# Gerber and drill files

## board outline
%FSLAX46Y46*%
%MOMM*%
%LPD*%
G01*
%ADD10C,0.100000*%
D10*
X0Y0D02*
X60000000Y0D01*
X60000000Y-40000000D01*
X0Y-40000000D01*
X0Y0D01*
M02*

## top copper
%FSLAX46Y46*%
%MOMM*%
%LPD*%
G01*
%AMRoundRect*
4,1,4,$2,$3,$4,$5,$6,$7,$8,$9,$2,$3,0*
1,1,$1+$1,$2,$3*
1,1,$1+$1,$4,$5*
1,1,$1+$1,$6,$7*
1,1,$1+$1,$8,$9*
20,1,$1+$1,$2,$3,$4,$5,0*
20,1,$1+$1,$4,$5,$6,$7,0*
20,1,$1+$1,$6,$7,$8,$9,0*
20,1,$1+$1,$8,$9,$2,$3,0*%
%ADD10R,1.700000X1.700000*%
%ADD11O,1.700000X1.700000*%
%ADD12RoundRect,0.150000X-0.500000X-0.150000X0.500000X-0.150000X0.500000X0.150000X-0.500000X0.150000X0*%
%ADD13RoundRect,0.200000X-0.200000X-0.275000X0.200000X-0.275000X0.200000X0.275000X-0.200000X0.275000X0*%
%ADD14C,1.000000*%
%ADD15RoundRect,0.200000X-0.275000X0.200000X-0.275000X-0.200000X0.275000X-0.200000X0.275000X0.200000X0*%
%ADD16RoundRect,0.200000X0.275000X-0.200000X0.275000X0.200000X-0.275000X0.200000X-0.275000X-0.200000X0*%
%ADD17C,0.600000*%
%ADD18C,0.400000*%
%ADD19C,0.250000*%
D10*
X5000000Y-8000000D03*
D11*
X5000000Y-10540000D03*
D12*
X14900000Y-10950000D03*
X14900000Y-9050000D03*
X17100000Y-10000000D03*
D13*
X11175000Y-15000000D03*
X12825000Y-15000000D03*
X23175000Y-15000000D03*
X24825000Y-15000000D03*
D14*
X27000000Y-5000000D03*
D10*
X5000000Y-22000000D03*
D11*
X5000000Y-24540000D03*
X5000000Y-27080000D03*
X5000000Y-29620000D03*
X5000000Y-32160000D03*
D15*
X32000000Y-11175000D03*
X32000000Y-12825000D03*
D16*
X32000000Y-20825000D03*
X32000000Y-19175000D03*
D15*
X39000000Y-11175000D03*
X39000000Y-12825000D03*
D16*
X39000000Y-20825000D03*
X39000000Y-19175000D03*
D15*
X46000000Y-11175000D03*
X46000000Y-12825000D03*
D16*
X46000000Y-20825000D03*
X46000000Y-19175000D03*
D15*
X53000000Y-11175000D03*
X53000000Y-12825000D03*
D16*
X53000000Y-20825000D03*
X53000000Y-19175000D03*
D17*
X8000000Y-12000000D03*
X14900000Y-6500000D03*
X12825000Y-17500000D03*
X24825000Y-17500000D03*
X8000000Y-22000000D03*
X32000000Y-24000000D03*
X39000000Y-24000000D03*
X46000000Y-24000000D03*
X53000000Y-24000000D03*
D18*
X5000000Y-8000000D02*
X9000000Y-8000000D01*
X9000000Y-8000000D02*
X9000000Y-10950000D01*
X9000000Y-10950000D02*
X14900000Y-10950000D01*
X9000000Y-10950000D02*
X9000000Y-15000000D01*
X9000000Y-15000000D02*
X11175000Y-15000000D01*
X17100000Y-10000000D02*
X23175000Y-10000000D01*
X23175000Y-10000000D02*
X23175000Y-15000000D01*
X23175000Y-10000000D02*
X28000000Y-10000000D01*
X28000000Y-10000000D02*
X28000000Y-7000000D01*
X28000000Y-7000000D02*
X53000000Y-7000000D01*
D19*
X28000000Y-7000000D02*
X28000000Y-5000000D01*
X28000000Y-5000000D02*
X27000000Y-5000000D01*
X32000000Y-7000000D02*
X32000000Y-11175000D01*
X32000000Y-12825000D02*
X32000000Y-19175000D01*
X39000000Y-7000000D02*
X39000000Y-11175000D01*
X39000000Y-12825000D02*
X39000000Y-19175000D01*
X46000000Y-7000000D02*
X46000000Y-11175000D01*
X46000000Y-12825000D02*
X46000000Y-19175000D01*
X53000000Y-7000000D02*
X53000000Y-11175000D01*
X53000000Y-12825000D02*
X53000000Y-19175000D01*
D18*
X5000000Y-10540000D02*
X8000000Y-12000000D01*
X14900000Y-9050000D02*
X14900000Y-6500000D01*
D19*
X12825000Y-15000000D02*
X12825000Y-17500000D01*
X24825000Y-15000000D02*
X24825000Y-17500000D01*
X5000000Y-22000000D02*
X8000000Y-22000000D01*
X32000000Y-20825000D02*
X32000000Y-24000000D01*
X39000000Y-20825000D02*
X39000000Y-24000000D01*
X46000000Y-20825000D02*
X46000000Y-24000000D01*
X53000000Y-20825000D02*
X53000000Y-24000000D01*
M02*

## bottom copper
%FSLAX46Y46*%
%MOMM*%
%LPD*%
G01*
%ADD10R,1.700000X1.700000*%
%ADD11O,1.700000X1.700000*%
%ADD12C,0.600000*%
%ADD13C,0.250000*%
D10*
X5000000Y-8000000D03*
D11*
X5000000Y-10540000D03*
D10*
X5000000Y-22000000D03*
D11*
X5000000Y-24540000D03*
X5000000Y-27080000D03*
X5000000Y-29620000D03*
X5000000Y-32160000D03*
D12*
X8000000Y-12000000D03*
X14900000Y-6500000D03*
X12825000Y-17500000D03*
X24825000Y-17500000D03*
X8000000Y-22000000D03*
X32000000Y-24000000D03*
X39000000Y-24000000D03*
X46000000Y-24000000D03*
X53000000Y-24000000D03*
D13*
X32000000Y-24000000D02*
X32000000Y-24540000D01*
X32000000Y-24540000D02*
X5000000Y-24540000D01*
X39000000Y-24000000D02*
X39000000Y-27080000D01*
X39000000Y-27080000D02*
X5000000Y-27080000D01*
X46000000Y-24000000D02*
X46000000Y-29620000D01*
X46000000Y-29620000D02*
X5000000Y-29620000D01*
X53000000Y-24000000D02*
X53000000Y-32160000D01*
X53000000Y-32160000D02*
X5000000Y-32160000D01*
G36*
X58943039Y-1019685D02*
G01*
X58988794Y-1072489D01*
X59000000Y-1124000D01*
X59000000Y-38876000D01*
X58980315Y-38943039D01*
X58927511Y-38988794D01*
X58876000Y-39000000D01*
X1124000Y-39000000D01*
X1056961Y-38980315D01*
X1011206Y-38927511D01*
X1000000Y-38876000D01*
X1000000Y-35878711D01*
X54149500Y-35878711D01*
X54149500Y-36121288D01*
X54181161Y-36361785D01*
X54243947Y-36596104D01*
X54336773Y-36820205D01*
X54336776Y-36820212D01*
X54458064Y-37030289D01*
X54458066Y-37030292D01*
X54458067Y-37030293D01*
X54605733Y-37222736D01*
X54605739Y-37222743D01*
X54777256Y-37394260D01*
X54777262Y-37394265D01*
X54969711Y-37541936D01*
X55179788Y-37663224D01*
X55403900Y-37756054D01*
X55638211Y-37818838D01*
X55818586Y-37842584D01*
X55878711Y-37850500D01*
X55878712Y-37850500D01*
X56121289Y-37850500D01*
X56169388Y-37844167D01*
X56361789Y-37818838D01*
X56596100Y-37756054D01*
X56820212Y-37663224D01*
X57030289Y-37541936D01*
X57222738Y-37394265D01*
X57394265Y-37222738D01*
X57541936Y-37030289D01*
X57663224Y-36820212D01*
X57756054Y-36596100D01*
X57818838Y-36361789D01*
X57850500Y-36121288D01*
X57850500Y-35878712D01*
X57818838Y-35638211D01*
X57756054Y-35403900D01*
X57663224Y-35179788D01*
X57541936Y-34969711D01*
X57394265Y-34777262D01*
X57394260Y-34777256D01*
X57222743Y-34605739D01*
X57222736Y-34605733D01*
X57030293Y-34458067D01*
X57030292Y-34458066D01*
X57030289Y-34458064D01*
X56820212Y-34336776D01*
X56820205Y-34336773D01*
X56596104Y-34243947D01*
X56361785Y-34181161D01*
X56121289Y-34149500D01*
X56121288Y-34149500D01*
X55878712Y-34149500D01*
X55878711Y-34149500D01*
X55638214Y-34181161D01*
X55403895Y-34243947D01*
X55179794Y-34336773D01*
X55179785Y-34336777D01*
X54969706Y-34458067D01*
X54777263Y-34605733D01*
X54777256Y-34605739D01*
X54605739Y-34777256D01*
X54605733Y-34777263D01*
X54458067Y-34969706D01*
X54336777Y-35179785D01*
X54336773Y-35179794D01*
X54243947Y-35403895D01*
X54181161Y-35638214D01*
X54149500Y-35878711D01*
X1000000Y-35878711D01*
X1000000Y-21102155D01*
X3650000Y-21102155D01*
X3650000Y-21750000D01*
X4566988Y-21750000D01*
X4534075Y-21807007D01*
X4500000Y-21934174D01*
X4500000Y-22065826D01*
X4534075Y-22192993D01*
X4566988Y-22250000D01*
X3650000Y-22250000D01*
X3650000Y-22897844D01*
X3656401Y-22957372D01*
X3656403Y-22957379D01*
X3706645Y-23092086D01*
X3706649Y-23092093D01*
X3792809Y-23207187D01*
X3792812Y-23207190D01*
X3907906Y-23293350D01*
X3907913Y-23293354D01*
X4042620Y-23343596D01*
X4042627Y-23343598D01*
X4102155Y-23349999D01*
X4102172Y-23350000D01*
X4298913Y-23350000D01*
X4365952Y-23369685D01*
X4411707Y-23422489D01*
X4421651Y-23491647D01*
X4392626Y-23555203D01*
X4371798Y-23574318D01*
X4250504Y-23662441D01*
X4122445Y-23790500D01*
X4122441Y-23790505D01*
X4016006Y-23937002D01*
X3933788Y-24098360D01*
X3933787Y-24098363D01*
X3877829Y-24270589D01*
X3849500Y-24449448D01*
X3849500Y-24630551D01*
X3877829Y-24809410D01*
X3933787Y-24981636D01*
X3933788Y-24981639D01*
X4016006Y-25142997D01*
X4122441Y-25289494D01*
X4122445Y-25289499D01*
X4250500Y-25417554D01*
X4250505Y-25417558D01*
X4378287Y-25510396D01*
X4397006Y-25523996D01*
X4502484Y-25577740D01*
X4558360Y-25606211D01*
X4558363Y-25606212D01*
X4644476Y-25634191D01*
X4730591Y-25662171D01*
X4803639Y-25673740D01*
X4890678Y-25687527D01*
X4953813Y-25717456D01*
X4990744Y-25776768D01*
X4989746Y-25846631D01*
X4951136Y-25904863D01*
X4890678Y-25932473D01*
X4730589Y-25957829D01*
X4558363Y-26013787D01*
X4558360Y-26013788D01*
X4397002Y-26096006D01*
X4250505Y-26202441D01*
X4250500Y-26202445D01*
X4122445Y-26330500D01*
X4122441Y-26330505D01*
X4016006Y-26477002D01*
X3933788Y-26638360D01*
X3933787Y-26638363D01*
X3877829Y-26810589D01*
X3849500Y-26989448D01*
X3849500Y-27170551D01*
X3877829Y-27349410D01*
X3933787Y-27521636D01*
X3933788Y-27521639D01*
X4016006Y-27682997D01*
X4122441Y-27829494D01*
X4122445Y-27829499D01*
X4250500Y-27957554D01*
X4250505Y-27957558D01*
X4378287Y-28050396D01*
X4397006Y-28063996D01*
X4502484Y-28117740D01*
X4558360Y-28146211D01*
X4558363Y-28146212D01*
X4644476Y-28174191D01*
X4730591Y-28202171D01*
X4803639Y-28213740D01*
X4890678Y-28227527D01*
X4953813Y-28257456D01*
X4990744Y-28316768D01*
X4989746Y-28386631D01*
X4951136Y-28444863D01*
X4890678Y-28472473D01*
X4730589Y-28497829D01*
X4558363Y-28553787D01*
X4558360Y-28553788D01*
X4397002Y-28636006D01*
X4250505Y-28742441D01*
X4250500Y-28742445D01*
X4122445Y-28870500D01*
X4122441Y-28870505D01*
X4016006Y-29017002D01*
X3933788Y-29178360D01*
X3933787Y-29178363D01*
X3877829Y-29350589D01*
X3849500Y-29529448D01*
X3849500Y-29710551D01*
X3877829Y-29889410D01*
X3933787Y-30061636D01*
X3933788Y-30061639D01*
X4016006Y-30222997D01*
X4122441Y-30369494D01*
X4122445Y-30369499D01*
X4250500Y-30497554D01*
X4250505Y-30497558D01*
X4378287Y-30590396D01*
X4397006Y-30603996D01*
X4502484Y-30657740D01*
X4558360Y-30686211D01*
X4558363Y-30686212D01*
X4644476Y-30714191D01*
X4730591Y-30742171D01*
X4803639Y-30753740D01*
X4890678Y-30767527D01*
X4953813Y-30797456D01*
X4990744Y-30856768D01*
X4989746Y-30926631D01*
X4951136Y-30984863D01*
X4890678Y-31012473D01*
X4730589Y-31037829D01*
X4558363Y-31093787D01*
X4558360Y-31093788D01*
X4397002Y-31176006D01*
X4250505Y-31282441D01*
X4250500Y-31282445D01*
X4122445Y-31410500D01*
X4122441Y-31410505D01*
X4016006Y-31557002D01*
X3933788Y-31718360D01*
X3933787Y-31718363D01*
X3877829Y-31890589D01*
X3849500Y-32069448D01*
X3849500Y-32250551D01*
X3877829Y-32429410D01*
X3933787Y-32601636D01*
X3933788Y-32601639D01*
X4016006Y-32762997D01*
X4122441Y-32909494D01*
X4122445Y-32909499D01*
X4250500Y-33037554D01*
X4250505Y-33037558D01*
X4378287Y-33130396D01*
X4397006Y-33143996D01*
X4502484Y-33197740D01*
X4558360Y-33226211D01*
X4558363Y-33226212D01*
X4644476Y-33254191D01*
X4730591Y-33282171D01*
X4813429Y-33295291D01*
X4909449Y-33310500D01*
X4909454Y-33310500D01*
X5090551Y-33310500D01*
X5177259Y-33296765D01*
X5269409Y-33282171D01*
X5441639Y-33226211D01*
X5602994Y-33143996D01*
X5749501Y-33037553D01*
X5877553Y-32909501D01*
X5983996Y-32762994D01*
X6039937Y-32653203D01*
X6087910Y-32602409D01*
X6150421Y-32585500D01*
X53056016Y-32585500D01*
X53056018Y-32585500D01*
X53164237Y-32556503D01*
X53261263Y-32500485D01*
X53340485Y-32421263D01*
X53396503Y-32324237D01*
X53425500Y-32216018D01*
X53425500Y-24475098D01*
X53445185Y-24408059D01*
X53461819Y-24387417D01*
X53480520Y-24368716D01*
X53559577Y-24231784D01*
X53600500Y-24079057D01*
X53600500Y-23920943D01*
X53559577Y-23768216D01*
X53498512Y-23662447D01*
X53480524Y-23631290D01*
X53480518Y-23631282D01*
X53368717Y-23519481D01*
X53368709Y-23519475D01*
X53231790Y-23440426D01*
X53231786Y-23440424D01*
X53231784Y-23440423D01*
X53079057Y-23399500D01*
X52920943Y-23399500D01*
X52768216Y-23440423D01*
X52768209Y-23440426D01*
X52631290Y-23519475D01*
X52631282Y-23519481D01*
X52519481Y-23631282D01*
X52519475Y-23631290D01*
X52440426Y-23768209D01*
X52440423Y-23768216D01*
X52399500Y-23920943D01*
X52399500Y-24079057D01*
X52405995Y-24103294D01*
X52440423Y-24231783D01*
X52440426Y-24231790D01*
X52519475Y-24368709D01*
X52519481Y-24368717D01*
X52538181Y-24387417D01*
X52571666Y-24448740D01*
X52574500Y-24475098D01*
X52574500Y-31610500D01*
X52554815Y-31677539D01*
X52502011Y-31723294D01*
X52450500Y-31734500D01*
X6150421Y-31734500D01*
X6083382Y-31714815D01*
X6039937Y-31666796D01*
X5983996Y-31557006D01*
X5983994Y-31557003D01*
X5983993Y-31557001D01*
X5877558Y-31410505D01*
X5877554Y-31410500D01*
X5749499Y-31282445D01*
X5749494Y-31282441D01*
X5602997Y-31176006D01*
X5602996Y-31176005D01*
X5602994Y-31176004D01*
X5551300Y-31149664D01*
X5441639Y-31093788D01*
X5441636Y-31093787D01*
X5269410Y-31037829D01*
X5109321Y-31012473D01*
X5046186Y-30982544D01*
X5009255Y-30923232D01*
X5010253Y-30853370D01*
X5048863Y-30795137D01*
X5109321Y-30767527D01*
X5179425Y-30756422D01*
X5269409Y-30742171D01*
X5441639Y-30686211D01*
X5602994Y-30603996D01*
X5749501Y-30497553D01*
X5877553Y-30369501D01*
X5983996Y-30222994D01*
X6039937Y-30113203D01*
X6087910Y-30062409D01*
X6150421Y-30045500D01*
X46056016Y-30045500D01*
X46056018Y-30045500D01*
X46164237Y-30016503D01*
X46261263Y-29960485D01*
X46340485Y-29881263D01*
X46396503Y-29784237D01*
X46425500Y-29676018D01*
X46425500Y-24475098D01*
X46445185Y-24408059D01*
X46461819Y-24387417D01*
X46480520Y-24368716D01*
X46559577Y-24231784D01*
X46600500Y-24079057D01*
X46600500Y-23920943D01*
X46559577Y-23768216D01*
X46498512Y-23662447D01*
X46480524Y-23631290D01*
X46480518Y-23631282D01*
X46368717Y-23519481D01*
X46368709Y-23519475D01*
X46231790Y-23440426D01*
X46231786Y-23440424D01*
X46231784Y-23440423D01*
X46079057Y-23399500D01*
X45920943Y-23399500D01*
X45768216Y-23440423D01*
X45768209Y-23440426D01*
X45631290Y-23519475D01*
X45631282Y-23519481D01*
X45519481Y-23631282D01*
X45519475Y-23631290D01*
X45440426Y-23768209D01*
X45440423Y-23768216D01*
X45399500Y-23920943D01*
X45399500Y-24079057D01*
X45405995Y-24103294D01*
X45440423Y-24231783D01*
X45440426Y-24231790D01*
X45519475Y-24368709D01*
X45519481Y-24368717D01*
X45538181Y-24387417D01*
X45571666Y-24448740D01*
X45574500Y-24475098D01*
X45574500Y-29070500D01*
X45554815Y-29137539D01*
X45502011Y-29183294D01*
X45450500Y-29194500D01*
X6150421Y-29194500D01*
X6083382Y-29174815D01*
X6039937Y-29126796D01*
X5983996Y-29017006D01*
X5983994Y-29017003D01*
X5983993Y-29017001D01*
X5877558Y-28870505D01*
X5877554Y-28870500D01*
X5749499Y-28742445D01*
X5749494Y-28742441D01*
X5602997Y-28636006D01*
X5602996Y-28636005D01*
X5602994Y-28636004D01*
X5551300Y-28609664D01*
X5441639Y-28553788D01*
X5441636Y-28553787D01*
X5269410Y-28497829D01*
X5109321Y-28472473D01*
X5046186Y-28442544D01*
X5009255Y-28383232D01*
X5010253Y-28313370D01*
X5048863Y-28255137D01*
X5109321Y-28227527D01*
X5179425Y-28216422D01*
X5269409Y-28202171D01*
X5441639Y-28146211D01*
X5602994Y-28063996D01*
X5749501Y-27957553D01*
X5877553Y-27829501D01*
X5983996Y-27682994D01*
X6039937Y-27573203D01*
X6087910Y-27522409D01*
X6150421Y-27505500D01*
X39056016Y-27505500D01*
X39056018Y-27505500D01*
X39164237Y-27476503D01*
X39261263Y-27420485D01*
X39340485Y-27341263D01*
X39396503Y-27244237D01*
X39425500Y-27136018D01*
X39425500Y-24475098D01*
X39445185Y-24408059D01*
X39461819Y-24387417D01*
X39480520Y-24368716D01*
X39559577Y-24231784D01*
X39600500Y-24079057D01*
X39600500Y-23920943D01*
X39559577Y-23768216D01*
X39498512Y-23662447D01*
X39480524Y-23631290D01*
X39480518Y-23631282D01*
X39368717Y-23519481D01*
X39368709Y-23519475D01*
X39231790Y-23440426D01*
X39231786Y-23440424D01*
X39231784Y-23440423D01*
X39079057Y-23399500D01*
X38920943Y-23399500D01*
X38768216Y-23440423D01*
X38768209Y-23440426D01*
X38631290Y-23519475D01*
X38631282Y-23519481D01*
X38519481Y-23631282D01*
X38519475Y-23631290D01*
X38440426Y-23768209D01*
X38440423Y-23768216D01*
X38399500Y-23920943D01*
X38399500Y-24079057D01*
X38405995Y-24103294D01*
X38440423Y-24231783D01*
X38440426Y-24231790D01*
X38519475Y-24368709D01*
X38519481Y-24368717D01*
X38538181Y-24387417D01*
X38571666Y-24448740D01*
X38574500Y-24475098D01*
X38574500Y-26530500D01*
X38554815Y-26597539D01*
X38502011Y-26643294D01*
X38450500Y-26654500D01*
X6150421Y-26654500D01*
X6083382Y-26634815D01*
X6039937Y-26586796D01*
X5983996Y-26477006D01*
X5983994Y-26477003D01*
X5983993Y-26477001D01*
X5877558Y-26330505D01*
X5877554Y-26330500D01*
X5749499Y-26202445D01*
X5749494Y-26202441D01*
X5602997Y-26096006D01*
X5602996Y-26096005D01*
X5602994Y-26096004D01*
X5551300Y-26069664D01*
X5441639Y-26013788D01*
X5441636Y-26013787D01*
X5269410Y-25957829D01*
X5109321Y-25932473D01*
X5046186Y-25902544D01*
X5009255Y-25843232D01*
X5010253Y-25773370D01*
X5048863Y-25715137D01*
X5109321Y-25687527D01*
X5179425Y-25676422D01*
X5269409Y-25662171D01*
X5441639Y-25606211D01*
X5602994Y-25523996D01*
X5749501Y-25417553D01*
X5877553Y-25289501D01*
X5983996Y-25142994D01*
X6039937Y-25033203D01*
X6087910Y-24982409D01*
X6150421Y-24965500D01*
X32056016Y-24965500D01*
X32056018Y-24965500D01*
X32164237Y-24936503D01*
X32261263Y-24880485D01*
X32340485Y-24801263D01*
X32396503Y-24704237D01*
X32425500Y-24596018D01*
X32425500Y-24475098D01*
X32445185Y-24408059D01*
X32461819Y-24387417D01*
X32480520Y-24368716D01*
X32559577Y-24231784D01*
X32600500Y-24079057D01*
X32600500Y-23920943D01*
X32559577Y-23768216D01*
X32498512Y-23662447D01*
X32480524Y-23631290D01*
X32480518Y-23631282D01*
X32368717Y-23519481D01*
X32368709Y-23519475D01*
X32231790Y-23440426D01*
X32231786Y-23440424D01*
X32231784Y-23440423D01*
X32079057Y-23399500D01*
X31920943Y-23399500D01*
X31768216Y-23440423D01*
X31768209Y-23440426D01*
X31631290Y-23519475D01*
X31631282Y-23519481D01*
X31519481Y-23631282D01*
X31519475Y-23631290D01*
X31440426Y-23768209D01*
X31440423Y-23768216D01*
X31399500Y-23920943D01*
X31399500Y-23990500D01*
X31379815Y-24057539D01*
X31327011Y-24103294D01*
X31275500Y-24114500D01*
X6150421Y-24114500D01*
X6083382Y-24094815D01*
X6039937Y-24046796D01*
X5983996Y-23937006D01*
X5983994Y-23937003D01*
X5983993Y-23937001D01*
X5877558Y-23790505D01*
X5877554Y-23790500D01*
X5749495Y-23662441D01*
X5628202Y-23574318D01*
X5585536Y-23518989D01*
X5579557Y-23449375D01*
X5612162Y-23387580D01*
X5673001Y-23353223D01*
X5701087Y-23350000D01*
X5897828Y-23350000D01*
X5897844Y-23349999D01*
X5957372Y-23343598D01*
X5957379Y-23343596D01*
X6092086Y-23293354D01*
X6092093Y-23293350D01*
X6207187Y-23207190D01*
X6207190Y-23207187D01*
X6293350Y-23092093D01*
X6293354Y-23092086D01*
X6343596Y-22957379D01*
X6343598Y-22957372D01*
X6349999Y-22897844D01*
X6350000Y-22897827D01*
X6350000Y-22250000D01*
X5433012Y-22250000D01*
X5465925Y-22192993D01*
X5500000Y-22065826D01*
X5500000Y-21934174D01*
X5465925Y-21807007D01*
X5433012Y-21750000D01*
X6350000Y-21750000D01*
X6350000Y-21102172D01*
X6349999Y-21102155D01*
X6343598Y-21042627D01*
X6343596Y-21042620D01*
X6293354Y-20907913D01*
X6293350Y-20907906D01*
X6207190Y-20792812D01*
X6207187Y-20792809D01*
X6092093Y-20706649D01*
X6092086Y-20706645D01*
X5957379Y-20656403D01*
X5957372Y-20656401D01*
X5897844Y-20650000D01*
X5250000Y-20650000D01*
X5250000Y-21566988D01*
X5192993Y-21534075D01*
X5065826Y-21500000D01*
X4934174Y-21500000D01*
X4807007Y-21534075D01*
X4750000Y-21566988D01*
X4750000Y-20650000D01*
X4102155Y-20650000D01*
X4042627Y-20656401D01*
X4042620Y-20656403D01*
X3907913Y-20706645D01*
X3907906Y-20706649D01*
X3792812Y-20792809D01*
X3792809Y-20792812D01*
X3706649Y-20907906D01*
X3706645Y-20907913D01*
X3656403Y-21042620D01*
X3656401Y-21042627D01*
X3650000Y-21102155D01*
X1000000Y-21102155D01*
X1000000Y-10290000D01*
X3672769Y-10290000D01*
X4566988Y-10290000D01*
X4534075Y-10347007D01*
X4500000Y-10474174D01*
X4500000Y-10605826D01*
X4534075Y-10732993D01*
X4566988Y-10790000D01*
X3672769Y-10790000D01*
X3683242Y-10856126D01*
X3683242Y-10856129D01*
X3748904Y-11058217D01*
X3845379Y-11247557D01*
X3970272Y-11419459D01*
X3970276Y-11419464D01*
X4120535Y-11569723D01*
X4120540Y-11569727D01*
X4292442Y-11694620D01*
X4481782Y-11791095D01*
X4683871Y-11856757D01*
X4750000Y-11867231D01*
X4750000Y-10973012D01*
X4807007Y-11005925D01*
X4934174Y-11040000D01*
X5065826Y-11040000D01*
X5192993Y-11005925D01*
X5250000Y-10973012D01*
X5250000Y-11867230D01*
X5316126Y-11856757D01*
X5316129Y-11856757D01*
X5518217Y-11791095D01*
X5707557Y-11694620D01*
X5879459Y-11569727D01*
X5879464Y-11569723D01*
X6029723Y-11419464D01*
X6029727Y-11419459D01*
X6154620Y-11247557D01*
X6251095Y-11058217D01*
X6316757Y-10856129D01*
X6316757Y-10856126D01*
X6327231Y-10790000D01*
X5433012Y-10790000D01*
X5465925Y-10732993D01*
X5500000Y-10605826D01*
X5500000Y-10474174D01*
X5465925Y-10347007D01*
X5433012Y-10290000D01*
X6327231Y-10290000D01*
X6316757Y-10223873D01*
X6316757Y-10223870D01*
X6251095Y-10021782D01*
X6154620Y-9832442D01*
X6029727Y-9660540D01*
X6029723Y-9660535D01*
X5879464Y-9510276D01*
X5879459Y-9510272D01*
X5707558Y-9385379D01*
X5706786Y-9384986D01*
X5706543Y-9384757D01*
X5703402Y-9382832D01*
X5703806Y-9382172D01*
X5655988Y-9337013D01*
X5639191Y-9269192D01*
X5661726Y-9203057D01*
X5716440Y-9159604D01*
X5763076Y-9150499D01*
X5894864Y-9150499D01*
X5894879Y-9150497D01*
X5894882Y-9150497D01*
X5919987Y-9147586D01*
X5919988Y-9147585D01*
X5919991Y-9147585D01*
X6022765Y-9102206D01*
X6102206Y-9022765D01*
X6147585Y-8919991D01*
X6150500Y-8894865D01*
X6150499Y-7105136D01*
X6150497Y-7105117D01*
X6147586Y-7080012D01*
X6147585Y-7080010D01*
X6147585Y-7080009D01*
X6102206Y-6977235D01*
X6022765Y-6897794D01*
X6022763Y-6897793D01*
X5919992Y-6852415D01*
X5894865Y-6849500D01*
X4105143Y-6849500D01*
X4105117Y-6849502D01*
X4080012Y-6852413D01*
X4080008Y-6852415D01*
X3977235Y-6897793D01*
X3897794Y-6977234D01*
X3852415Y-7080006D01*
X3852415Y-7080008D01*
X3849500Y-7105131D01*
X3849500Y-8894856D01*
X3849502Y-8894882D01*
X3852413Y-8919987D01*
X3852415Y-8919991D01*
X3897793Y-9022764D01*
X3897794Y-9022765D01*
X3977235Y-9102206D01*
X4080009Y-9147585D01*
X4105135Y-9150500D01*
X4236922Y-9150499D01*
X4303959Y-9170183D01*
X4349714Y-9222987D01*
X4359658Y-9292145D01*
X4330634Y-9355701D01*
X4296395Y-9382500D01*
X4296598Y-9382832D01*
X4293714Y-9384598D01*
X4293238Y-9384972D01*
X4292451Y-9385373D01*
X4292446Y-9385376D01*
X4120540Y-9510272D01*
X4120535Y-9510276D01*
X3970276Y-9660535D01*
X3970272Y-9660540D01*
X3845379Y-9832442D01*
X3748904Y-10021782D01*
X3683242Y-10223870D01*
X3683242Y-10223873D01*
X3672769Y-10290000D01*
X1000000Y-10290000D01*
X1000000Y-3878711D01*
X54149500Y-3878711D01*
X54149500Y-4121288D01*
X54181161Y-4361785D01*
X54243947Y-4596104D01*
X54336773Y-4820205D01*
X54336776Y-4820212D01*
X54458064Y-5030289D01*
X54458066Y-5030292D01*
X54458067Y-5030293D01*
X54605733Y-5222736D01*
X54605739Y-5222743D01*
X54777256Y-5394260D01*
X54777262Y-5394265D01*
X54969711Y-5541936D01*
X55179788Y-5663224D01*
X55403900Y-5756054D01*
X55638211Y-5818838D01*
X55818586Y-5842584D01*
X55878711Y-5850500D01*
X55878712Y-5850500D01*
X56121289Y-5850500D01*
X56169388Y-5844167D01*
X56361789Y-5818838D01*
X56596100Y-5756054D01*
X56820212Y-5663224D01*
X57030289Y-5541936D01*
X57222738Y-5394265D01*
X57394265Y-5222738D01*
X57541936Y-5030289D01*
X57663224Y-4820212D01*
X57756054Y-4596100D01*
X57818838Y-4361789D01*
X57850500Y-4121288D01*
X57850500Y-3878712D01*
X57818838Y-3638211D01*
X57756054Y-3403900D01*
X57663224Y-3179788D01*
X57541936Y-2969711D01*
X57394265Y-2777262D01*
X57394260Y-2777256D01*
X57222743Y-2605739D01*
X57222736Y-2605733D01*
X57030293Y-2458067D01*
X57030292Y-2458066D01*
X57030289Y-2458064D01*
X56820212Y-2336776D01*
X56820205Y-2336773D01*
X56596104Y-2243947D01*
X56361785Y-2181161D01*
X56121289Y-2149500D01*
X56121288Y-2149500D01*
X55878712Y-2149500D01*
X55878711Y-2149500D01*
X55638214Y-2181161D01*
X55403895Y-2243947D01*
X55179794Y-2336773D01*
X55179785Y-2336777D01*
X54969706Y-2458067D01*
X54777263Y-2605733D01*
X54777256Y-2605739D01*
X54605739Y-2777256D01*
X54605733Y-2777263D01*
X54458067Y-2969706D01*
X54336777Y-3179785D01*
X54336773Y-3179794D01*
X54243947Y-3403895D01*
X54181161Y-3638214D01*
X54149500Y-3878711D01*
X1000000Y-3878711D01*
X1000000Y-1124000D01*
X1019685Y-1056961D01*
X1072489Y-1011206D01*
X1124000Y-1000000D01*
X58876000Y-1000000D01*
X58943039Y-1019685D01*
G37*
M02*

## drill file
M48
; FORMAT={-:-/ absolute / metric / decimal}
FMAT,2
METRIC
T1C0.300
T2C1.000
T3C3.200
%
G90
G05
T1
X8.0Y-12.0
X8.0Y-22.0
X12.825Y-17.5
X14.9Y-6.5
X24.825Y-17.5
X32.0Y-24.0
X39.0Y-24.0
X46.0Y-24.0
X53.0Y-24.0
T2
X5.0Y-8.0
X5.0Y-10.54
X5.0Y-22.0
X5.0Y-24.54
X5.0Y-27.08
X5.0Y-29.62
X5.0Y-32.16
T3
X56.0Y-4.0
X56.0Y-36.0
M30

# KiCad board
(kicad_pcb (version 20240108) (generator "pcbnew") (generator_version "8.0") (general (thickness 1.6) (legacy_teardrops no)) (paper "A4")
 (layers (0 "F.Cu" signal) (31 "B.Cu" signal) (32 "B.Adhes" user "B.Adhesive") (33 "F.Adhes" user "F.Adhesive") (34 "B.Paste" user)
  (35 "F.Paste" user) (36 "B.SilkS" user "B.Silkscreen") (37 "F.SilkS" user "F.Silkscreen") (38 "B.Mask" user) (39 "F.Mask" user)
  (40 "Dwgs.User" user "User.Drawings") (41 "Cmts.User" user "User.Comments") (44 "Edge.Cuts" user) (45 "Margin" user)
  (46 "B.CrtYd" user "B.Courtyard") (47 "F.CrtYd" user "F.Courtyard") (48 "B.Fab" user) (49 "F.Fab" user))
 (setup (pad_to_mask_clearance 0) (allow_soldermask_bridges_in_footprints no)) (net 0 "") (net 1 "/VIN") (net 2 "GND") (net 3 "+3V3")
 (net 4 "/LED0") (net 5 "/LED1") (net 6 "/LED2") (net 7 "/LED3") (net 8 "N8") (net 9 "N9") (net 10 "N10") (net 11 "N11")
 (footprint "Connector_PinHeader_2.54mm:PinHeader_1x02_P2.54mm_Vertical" (layer "F.Cu") (at 5 8)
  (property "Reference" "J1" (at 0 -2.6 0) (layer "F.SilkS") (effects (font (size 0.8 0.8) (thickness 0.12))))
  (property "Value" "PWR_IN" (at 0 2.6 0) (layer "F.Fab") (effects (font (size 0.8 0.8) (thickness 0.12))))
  (pad "1" thru_hole rect (at 0 0) (size 1.7 1.7) (drill 1) (layers "*.Cu" "*.Mask") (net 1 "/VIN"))
  (pad "2" thru_hole oval (at 0 2.54) (size 1.7 1.7) (drill 1) (layers "*.Cu" "*.Mask") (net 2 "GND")))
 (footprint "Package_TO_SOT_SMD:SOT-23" (layer "F.Cu") (at 16 10)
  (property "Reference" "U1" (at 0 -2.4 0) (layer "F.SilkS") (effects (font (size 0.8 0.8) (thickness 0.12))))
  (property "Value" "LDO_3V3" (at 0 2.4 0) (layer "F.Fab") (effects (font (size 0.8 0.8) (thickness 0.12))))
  (pad "1" smd roundrect (at -1.1 0.95) (size 1.3 0.6) (layers "F.Cu" "F.Paste" "F.Mask") (roundrect_rratio 0.25) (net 1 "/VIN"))
  (pad "2" smd roundrect (at -1.1 -0.95) (size 1.3 0.6) (layers "F.Cu" "F.Paste" "F.Mask") (roundrect_rratio 0.25) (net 2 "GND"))
  (pad "3" smd roundrect (at 1.1 0) (size 1.3 0.6) (layers "F.Cu" "F.Paste" "F.Mask") (roundrect_rratio 0.25) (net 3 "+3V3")))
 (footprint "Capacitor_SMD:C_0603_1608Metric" (layer "F.Cu") (at 12 15)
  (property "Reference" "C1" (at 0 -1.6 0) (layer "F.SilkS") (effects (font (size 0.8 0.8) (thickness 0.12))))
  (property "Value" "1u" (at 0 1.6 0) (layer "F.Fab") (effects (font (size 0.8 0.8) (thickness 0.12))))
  (pad "1" smd roundrect (at -0.825 0) (size 0.8 0.95) (layers "F.Cu" "F.Paste" "F.Mask") (roundrect_rratio 0.25) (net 1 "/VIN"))
  (pad "2" smd roundrect (at 0.825 0) (size 0.8 0.95) (layers "F.Cu" "F.Paste" "F.Mask") (roundrect_rratio 0.25) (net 2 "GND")))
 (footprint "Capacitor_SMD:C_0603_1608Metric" (layer "F.Cu") (at 24 15)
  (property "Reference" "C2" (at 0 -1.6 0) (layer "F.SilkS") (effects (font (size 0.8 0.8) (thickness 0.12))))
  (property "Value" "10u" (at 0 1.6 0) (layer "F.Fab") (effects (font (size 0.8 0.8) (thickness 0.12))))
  (pad "1" smd roundrect (at -0.825 0) (size 0.8 0.95) (layers "F.Cu" "F.Paste" "F.Mask") (roundrect_rratio 0.25) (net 3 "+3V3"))
  (pad "2" smd roundrect (at 0.825 0) (size 0.8 0.95) (layers "F.Cu" "F.Paste" "F.Mask") (roundrect_rratio 0.25) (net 2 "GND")))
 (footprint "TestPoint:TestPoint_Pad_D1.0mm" (layer "F.Cu") (at 27 5)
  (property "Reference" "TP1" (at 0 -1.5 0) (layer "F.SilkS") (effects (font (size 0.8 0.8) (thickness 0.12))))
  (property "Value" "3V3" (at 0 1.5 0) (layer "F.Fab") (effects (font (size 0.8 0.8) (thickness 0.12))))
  (pad "1" smd circle (at 0 0) (size 1 1) (layers "F.Cu" "F.Mask") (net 3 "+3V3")))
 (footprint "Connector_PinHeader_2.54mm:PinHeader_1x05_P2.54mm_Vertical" (layer "F.Cu") (at 5 22)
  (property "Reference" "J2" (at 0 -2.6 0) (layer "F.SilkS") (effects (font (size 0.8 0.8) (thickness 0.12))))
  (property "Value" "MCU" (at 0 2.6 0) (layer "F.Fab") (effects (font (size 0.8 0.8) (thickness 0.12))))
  (pad "1" thru_hole rect (at 0 0) (size 1.7 1.7) (drill 1) (layers "*.Cu" "*.Mask") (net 2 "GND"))
  (pad "2" thru_hole oval (at 0 2.54) (size 1.7 1.7) (drill 1) (layers "*.Cu" "*.Mask") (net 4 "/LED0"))
  (pad "3" thru_hole oval (at 0 5.08) (size 1.7 1.7) (drill 1) (layers "*.Cu" "*.Mask") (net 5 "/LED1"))
  (pad "4" thru_hole oval (at 0 7.62) (size 1.7 1.7) (drill 1) (layers "*.Cu" "*.Mask") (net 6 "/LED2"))
  (pad "5" thru_hole oval (at 0 10.16) (size 1.7 1.7) (drill 1) (layers "*.Cu" "*.Mask") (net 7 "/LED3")))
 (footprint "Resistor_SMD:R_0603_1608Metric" (layer "F.Cu") (at 32 12 270)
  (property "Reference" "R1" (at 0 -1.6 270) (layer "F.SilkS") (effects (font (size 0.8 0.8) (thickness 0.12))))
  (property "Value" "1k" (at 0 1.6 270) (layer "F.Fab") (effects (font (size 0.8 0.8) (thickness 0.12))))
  (pad "1" smd roundrect (at -0.825 0 270) (size 0.8 0.95) (layers "F.Cu" "F.Paste" "F.Mask") (roundrect_rratio 0.25) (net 3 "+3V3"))
  (pad "2" smd roundrect (at 0.825 0 270) (size 0.8 0.95) (layers "F.Cu" "F.Paste" "F.Mask") (roundrect_rratio 0.25) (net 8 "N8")))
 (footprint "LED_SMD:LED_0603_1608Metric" (layer "F.Cu") (at 32 20 90)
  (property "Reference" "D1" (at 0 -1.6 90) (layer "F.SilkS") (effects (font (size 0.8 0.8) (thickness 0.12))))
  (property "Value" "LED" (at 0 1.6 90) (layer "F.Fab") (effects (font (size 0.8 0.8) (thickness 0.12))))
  (pad "1" smd roundrect (at -0.825 0 90) (size 0.8 0.95) (layers "F.Cu" "F.Paste" "F.Mask") (roundrect_rratio 0.25) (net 4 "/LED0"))
  (pad "2" smd roundrect (at 0.825 0 90) (size 0.8 0.95) (layers "F.Cu" "F.Paste" "F.Mask") (roundrect_rratio 0.25) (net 8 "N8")))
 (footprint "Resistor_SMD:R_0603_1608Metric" (layer "F.Cu") (at 39 12 270)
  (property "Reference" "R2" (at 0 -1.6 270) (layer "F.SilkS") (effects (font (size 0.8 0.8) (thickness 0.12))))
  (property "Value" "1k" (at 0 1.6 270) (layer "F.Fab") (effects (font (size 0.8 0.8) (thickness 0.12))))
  (pad "1" smd roundrect (at -0.825 0 270) (size 0.8 0.95) (layers "F.Cu" "F.Paste" "F.Mask") (roundrect_rratio 0.25) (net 3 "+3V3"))
  (pad "2" smd roundrect (at 0.825 0 270) (size 0.8 0.95) (layers "F.Cu" "F.Paste" "F.Mask") (roundrect_rratio 0.25) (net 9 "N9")))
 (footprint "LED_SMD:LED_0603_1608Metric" (layer "F.Cu") (at 39 20 90)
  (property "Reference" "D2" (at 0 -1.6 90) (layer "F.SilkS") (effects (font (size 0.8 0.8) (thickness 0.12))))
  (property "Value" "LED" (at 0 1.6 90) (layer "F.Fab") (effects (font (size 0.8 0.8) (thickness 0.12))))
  (pad "1" smd roundrect (at -0.825 0 90) (size 0.8 0.95) (layers "F.Cu" "F.Paste" "F.Mask") (roundrect_rratio 0.25) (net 5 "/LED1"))
  (pad "2" smd roundrect (at 0.825 0 90) (size 0.8 0.95) (layers "F.Cu" "F.Paste" "F.Mask") (roundrect_rratio 0.25) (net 9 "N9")))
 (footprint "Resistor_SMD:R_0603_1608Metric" (layer "F.Cu") (at 46 12 270)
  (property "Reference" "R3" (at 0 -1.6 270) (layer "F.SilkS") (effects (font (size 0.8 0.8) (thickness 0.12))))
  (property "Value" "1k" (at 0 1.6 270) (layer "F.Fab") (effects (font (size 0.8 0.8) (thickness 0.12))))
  (pad "1" smd roundrect (at -0.825 0 270) (size 0.8 0.95) (layers "F.Cu" "F.Paste" "F.Mask") (roundrect_rratio 0.25) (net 3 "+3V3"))
  (pad "2" smd roundrect (at 0.825 0 270) (size 0.8 0.95) (layers "F.Cu" "F.Paste" "F.Mask") (roundrect_rratio 0.25) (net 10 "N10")))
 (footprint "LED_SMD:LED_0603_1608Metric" (layer "F.Cu") (at 46 20 90)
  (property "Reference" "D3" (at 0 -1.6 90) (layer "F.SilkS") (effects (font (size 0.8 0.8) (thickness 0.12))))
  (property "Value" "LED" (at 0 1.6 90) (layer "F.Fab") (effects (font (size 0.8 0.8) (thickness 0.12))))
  (pad "1" smd roundrect (at -0.825 0 90) (size 0.8 0.95) (layers "F.Cu" "F.Paste" "F.Mask") (roundrect_rratio 0.25) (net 6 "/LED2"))
  (pad "2" smd roundrect (at 0.825 0 90) (size 0.8 0.95) (layers "F.Cu" "F.Paste" "F.Mask") (roundrect_rratio 0.25) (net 10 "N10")))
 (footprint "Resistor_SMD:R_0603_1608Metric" (layer "F.Cu") (at 53 12 270)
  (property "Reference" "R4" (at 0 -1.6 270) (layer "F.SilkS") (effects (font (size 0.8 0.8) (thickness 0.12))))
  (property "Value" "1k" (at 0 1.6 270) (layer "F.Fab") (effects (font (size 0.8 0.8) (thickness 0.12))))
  (pad "1" smd roundrect (at -0.825 0 270) (size 0.8 0.95) (layers "F.Cu" "F.Paste" "F.Mask") (roundrect_rratio 0.25) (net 3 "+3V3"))
  (pad "2" smd roundrect (at 0.825 0 270) (size 0.8 0.95) (layers "F.Cu" "F.Paste" "F.Mask") (roundrect_rratio 0.25) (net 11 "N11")))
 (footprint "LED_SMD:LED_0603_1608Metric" (layer "F.Cu") (at 53 20 90)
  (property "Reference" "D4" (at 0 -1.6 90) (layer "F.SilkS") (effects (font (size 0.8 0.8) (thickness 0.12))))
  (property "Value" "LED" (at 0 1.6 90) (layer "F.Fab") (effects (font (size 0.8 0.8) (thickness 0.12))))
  (pad "1" smd roundrect (at -0.825 0 90) (size 0.8 0.95) (layers "F.Cu" "F.Paste" "F.Mask") (roundrect_rratio 0.25) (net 7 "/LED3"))
  (pad "2" smd roundrect (at 0.825 0 90) (size 0.8 0.95) (layers "F.Cu" "F.Paste" "F.Mask") (roundrect_rratio 0.25) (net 11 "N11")))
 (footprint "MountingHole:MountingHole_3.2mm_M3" (layer "F.Cu") (at 56 4)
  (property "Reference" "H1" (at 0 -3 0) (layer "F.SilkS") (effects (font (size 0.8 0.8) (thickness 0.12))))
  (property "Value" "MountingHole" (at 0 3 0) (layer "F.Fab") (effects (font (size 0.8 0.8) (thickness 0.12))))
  (pad "" np_thru_hole circle (at 0 0) (size 3.2 3.2) (drill 3.2) (layers "*.Cu" "*.Mask")))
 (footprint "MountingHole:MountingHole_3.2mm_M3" (layer "F.Cu") (at 56 36)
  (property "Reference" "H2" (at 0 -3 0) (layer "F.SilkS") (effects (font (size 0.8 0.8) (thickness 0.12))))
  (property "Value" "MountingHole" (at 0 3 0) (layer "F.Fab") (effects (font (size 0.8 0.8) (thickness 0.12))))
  (pad "" np_thru_hole circle (at 0 0) (size 3.2 3.2) (drill 3.2) (layers "*.Cu" "*.Mask")))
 (segment (start 5 8) (end 9 8) (width 0.4) (layer "F.Cu") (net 1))
 (segment (start 9 8) (end 9 10.95) (width 0.4) (layer "F.Cu") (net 1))
 (segment (start 9 10.95) (end 14.9 10.95) (width 0.4) (layer "F.Cu") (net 1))
 (segment (start 9 10.95) (end 9 15) (width 0.4) (layer "F.Cu") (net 1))
 (segment (start 9 15) (end 11.175 15) (width 0.4) (layer "F.Cu") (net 1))
 (segment (start 17.1 10) (end 23.175 10) (width 0.4) (layer "F.Cu") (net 3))
 (segment (start 23.175 10) (end 23.175 15) (width 0.4) (layer "F.Cu") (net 3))
 (segment (start 23.175 10) (end 28 10) (width 0.4) (layer "F.Cu") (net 3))
 (segment (start 28 10) (end 28 7) (width 0.4) (layer "F.Cu") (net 3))
 (segment (start 28 7) (end 53 7) (width 0.4) (layer "F.Cu") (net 3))
 (segment (start 28 7) (end 28 5) (width 0.25) (layer "F.Cu") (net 3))
 (segment (start 28 5) (end 27 5) (width 0.25) (layer "F.Cu") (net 3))
 (segment (start 32 7) (end 32 11.175) (width 0.25) (layer "F.Cu") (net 3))
 (segment (start 32 12.825) (end 32 19.175) (width 0.25) (layer "F.Cu") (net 8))
 (segment (start 39 7) (end 39 11.175) (width 0.25) (layer "F.Cu") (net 3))
 (segment (start 39 12.825) (end 39 19.175) (width 0.25) (layer "F.Cu") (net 9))
 (segment (start 46 7) (end 46 11.175) (width 0.25) (layer "F.Cu") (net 3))
 (segment (start 46 12.825) (end 46 19.175) (width 0.25) (layer "F.Cu") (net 10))
 (segment (start 53 7) (end 53 11.175) (width 0.25) (layer "F.Cu") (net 3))
 (segment (start 53 12.825) (end 53 19.175) (width 0.25) (layer "F.Cu") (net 11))
 (segment (start 5 10.54) (end 8 12) (width 0.4) (layer "F.Cu") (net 2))
 (via (at 8 12) (size 0.6) (drill 0.3) (layers "F.Cu" "B.Cu") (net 2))
 (segment (start 14.9 9.05) (end 14.9 6.5) (width 0.4) (layer "F.Cu") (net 2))
 (via (at 14.9 6.5) (size 0.6) (drill 0.3) (layers "F.Cu" "B.Cu") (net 2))
 (segment (start 12.825 15) (end 12.825 17.5) (width 0.25) (layer "F.Cu") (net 2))
 (via (at 12.825 17.5) (size 0.6) (drill 0.3) (layers "F.Cu" "B.Cu") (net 2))
 (segment (start 24.825 15) (end 24.825 17.5) (width 0.25) (layer "F.Cu") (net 2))
 (via (at 24.825 17.5) (size 0.6) (drill 0.3) (layers "F.Cu" "B.Cu") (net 2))
 (segment (start 5 22) (end 8 22) (width 0.25) (layer "F.Cu") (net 2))
 (via (at 8 22) (size 0.6) (drill 0.3) (layers "F.Cu" "B.Cu") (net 2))
 (segment (start 32 20.825) (end 32 24) (width 0.25) (layer "F.Cu") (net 4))
 (via (at 32 24) (size 0.6) (drill 0.3) (layers "F.Cu" "B.Cu") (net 4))
 (segment (start 32 24) (end 32 24.54) (width 0.25) (layer "B.Cu") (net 4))
 (segment (start 32 24.54) (end 5 24.54) (width 0.25) (layer "B.Cu") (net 4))
 (segment (start 39 20.825) (end 39 24) (width 0.25) (layer "F.Cu") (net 5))
 (via (at 39 24) (size 0.6) (drill 0.3) (layers "F.Cu" "B.Cu") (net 5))
 (segment (start 39 24) (end 39 27.08) (width 0.25) (layer "B.Cu") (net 5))
 (segment (start 39 27.08) (end 5 27.08) (width 0.25) (layer "B.Cu") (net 5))
 (segment (start 46 20.825) (end 46 24) (width 0.25) (layer "F.Cu") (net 6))
 (via (at 46 24) (size 0.6) (drill 0.3) (layers "F.Cu" "B.Cu") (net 6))
 (segment (start 46 24) (end 46 29.62) (width 0.25) (layer "B.Cu") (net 6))
 (segment (start 46 29.62) (end 5 29.62) (width 0.25) (layer "B.Cu") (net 6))
 (segment (start 53 20.825) (end 53 24) (width 0.25) (layer "F.Cu") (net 7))
 (via (at 53 24) (size 0.6) (drill 0.3) (layers "F.Cu" "B.Cu") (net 7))
 (segment (start 53 24) (end 53 32.16) (width 0.25) (layer "B.Cu") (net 7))
 (segment (start 53 32.16) (end 5 32.16) (width 0.25) (layer "B.Cu") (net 7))
 (gr_rect (start 0 0) (end 60 40) (stroke (width 0.1) (type default)) (fill none) (layer "Edge.Cuts"))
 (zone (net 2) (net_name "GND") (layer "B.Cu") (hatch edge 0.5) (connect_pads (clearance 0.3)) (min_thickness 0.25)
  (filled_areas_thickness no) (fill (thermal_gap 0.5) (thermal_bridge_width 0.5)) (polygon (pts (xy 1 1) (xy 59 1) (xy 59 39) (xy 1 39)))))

